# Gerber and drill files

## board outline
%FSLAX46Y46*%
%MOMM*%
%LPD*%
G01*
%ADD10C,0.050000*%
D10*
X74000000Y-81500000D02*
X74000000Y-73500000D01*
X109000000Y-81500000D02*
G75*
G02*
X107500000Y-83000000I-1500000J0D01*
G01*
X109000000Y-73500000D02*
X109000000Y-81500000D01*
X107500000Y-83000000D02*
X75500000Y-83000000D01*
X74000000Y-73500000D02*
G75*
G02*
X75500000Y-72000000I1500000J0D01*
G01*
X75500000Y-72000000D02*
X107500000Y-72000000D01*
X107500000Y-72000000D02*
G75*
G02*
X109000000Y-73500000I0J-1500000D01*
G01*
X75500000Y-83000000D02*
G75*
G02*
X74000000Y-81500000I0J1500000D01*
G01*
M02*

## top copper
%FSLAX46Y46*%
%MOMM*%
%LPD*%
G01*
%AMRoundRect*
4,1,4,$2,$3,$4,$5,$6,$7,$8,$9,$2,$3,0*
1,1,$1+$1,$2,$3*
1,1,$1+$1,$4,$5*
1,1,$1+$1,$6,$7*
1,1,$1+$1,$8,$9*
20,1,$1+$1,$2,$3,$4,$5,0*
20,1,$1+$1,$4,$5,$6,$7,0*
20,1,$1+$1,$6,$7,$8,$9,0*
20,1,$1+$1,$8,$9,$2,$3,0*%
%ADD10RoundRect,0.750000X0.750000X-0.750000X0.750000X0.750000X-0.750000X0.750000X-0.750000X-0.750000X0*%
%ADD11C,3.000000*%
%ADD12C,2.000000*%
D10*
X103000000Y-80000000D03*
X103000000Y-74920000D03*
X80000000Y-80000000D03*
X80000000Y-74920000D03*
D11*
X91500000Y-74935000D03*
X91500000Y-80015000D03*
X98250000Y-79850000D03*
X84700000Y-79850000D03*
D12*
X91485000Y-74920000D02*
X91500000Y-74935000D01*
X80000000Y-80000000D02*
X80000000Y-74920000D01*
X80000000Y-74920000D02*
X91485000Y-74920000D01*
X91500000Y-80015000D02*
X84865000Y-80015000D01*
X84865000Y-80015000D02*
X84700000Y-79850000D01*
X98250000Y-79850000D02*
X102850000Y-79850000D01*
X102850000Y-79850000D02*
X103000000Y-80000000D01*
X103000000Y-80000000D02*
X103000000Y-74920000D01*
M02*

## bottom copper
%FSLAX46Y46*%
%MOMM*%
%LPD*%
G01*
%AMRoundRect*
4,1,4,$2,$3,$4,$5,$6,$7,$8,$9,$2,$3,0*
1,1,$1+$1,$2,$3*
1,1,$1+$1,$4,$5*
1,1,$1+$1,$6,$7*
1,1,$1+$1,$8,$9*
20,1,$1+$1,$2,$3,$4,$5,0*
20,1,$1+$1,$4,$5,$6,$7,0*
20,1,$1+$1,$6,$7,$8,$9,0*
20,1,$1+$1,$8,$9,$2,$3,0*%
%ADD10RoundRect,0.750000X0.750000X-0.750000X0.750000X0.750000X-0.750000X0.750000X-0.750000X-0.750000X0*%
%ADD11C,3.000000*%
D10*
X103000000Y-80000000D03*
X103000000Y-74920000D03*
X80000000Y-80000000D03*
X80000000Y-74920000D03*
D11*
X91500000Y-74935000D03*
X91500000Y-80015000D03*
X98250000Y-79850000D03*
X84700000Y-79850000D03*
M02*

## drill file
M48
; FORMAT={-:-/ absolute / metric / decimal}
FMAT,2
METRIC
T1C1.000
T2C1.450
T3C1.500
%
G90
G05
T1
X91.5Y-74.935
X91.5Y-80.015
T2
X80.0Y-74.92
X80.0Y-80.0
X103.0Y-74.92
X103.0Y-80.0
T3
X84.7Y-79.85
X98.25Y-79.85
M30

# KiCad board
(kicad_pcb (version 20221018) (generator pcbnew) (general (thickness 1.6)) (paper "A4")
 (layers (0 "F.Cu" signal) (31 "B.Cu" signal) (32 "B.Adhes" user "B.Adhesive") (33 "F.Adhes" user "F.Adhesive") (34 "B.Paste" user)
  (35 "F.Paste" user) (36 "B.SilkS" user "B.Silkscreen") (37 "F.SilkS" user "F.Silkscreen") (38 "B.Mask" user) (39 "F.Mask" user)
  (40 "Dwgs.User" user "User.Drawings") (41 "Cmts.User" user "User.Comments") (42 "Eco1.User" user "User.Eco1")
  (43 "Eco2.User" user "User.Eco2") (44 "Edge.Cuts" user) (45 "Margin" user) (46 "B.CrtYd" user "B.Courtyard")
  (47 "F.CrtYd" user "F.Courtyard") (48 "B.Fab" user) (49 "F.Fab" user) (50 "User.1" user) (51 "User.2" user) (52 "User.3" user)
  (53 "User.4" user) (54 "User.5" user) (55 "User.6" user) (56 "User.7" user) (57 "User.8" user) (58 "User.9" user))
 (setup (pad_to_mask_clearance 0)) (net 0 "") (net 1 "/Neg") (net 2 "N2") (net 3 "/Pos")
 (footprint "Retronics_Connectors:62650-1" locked (layer "F.Cu") (at 103 80 90)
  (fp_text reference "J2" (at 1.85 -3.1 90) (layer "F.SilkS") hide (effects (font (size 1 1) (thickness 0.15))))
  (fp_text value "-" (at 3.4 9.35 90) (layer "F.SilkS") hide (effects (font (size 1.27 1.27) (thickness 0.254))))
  (pad "1" thru_hole roundrect locked (at 0 0 90) (size 3 3) (drill 1.45) (layers "*.Cu" "*.Mask") (roundrect_rratio 0.25) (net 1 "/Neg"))
  (pad "1" thru_hole roundrect locked (at 5.08 0 90) (size 3 3) (drill 1.45) (layers "*.Cu" "*.Mask") (roundrect_rratio 0.25) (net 1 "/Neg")))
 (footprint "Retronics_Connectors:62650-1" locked (layer "F.Cu") (at 80 80 90)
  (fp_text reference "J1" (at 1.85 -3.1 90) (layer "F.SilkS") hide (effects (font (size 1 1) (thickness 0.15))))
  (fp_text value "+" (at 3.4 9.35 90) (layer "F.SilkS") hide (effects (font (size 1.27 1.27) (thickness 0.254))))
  (pad "1" thru_hole roundrect locked (at 0 0 90) (size 3 3) (drill 1.45) (layers "*.Cu" "*.Mask") (roundrect_rratio 0.25) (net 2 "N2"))
  (pad "1" thru_hole roundrect locked (at 5.08 0 90) (size 3 3) (drill 1.45) (layers "*.Cu" "*.Mask") (roundrect_rratio 0.25) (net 2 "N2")))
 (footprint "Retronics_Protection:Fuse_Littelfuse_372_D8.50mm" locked (layer "B.Cu") (at 91.5 74.935 -90)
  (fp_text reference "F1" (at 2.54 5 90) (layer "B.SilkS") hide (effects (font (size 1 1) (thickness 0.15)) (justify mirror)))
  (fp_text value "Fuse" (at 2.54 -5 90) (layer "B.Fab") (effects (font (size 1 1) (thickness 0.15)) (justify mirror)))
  (pad "1" thru_hole circle locked (at 0 0 270) (size 3 3) (drill 1) (layers "*.Cu" "*.Mask") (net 2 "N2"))
  (pad "2" thru_hole circle locked (at 5.08 0 270) (size 3 3) (drill 1) (layers "*.Cu" "*.Mask") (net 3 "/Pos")))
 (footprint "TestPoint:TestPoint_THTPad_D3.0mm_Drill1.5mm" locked (layer "B.Cu") (at 98.25 79.85 180)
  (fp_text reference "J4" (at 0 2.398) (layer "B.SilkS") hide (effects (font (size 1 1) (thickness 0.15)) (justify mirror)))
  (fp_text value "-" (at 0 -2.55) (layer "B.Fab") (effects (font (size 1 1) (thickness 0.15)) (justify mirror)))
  (pad "1" thru_hole circle locked (at 0 0 180) (size 3 3) (drill 1.5) (layers "*.Cu" "*.Mask") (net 1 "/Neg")))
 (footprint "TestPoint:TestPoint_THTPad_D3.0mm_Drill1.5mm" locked (layer "B.Cu") (at 84.7 79.85 180)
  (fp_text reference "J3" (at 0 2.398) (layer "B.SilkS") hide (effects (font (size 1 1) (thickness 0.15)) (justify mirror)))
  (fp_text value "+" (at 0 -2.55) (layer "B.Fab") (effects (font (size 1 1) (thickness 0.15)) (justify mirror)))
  (pad "1" thru_hole circle locked (at 0 0 180) (size 3 3) (drill 1.5) (layers "*.Cu" "*.Mask") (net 3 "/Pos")))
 (gr_line (start 74 81.5) (end 74 73.5) (stroke (width 0.05) (type default)) (layer "Edge.Cuts"))
 (gr_arc (start 109 81.5) (mid 108.56066 82.56066) (end 107.5 83) (stroke (width 0.05) (type default)) (layer "Edge.Cuts"))
 (gr_line (start 109 73.5) (end 109 81.5) (stroke (width 0.05) (type default)) (layer "Edge.Cuts"))
 (gr_line (start 107.5 83) (end 75.5 83) (stroke (width 0.05) (type default)) (layer "Edge.Cuts"))
 (gr_arc (start 74 73.5) (mid 74.43934 72.43934) (end 75.5 72) (stroke (width 0.05) (type default)) (layer "Edge.Cuts"))
 (gr_line (start 75.5 72) (end 107.5 72) (stroke (width 0.05) (type default)) (layer "Edge.Cuts"))
 (gr_arc (start 107.5 72) (mid 108.56066 72.43934) (end 109 73.5) (stroke (width 0.05) (type default)) (layer "Edge.Cuts"))
 (gr_arc (start 75.5 83) (mid 74.43934 82.56066) (end 74 81.5) (stroke (width 0.05) (type default)) (layer "Edge.Cuts"))
 (segment (start 91.485 74.92) (end 91.5 74.935) (width 2) (layer "F.Cu") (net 2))
 (segment (start 80 80) (end 80 74.92) (width 2) (layer "F.Cu") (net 2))
 (segment (start 80 74.92) (end 91.485 74.92) (width 2) (layer "F.Cu") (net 2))
 (segment (start 91.5 80.015) (end 84.865 80.015) (width 2) (layer "F.Cu") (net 3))
 (segment (start 84.865 80.015) (end 84.7 79.85) (width 2) (layer "F.Cu") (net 3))
 (segment (start 98.25 79.85) (end 102.85 79.85) (width 2) (layer "F.Cu") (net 1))
 (segment (start 102.85 79.85) (end 103 80) (width 2) (layer "F.Cu") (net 1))
 (segment (start 103 80) (end 103 74.92) (width 2) (layer "F.Cu") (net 1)))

